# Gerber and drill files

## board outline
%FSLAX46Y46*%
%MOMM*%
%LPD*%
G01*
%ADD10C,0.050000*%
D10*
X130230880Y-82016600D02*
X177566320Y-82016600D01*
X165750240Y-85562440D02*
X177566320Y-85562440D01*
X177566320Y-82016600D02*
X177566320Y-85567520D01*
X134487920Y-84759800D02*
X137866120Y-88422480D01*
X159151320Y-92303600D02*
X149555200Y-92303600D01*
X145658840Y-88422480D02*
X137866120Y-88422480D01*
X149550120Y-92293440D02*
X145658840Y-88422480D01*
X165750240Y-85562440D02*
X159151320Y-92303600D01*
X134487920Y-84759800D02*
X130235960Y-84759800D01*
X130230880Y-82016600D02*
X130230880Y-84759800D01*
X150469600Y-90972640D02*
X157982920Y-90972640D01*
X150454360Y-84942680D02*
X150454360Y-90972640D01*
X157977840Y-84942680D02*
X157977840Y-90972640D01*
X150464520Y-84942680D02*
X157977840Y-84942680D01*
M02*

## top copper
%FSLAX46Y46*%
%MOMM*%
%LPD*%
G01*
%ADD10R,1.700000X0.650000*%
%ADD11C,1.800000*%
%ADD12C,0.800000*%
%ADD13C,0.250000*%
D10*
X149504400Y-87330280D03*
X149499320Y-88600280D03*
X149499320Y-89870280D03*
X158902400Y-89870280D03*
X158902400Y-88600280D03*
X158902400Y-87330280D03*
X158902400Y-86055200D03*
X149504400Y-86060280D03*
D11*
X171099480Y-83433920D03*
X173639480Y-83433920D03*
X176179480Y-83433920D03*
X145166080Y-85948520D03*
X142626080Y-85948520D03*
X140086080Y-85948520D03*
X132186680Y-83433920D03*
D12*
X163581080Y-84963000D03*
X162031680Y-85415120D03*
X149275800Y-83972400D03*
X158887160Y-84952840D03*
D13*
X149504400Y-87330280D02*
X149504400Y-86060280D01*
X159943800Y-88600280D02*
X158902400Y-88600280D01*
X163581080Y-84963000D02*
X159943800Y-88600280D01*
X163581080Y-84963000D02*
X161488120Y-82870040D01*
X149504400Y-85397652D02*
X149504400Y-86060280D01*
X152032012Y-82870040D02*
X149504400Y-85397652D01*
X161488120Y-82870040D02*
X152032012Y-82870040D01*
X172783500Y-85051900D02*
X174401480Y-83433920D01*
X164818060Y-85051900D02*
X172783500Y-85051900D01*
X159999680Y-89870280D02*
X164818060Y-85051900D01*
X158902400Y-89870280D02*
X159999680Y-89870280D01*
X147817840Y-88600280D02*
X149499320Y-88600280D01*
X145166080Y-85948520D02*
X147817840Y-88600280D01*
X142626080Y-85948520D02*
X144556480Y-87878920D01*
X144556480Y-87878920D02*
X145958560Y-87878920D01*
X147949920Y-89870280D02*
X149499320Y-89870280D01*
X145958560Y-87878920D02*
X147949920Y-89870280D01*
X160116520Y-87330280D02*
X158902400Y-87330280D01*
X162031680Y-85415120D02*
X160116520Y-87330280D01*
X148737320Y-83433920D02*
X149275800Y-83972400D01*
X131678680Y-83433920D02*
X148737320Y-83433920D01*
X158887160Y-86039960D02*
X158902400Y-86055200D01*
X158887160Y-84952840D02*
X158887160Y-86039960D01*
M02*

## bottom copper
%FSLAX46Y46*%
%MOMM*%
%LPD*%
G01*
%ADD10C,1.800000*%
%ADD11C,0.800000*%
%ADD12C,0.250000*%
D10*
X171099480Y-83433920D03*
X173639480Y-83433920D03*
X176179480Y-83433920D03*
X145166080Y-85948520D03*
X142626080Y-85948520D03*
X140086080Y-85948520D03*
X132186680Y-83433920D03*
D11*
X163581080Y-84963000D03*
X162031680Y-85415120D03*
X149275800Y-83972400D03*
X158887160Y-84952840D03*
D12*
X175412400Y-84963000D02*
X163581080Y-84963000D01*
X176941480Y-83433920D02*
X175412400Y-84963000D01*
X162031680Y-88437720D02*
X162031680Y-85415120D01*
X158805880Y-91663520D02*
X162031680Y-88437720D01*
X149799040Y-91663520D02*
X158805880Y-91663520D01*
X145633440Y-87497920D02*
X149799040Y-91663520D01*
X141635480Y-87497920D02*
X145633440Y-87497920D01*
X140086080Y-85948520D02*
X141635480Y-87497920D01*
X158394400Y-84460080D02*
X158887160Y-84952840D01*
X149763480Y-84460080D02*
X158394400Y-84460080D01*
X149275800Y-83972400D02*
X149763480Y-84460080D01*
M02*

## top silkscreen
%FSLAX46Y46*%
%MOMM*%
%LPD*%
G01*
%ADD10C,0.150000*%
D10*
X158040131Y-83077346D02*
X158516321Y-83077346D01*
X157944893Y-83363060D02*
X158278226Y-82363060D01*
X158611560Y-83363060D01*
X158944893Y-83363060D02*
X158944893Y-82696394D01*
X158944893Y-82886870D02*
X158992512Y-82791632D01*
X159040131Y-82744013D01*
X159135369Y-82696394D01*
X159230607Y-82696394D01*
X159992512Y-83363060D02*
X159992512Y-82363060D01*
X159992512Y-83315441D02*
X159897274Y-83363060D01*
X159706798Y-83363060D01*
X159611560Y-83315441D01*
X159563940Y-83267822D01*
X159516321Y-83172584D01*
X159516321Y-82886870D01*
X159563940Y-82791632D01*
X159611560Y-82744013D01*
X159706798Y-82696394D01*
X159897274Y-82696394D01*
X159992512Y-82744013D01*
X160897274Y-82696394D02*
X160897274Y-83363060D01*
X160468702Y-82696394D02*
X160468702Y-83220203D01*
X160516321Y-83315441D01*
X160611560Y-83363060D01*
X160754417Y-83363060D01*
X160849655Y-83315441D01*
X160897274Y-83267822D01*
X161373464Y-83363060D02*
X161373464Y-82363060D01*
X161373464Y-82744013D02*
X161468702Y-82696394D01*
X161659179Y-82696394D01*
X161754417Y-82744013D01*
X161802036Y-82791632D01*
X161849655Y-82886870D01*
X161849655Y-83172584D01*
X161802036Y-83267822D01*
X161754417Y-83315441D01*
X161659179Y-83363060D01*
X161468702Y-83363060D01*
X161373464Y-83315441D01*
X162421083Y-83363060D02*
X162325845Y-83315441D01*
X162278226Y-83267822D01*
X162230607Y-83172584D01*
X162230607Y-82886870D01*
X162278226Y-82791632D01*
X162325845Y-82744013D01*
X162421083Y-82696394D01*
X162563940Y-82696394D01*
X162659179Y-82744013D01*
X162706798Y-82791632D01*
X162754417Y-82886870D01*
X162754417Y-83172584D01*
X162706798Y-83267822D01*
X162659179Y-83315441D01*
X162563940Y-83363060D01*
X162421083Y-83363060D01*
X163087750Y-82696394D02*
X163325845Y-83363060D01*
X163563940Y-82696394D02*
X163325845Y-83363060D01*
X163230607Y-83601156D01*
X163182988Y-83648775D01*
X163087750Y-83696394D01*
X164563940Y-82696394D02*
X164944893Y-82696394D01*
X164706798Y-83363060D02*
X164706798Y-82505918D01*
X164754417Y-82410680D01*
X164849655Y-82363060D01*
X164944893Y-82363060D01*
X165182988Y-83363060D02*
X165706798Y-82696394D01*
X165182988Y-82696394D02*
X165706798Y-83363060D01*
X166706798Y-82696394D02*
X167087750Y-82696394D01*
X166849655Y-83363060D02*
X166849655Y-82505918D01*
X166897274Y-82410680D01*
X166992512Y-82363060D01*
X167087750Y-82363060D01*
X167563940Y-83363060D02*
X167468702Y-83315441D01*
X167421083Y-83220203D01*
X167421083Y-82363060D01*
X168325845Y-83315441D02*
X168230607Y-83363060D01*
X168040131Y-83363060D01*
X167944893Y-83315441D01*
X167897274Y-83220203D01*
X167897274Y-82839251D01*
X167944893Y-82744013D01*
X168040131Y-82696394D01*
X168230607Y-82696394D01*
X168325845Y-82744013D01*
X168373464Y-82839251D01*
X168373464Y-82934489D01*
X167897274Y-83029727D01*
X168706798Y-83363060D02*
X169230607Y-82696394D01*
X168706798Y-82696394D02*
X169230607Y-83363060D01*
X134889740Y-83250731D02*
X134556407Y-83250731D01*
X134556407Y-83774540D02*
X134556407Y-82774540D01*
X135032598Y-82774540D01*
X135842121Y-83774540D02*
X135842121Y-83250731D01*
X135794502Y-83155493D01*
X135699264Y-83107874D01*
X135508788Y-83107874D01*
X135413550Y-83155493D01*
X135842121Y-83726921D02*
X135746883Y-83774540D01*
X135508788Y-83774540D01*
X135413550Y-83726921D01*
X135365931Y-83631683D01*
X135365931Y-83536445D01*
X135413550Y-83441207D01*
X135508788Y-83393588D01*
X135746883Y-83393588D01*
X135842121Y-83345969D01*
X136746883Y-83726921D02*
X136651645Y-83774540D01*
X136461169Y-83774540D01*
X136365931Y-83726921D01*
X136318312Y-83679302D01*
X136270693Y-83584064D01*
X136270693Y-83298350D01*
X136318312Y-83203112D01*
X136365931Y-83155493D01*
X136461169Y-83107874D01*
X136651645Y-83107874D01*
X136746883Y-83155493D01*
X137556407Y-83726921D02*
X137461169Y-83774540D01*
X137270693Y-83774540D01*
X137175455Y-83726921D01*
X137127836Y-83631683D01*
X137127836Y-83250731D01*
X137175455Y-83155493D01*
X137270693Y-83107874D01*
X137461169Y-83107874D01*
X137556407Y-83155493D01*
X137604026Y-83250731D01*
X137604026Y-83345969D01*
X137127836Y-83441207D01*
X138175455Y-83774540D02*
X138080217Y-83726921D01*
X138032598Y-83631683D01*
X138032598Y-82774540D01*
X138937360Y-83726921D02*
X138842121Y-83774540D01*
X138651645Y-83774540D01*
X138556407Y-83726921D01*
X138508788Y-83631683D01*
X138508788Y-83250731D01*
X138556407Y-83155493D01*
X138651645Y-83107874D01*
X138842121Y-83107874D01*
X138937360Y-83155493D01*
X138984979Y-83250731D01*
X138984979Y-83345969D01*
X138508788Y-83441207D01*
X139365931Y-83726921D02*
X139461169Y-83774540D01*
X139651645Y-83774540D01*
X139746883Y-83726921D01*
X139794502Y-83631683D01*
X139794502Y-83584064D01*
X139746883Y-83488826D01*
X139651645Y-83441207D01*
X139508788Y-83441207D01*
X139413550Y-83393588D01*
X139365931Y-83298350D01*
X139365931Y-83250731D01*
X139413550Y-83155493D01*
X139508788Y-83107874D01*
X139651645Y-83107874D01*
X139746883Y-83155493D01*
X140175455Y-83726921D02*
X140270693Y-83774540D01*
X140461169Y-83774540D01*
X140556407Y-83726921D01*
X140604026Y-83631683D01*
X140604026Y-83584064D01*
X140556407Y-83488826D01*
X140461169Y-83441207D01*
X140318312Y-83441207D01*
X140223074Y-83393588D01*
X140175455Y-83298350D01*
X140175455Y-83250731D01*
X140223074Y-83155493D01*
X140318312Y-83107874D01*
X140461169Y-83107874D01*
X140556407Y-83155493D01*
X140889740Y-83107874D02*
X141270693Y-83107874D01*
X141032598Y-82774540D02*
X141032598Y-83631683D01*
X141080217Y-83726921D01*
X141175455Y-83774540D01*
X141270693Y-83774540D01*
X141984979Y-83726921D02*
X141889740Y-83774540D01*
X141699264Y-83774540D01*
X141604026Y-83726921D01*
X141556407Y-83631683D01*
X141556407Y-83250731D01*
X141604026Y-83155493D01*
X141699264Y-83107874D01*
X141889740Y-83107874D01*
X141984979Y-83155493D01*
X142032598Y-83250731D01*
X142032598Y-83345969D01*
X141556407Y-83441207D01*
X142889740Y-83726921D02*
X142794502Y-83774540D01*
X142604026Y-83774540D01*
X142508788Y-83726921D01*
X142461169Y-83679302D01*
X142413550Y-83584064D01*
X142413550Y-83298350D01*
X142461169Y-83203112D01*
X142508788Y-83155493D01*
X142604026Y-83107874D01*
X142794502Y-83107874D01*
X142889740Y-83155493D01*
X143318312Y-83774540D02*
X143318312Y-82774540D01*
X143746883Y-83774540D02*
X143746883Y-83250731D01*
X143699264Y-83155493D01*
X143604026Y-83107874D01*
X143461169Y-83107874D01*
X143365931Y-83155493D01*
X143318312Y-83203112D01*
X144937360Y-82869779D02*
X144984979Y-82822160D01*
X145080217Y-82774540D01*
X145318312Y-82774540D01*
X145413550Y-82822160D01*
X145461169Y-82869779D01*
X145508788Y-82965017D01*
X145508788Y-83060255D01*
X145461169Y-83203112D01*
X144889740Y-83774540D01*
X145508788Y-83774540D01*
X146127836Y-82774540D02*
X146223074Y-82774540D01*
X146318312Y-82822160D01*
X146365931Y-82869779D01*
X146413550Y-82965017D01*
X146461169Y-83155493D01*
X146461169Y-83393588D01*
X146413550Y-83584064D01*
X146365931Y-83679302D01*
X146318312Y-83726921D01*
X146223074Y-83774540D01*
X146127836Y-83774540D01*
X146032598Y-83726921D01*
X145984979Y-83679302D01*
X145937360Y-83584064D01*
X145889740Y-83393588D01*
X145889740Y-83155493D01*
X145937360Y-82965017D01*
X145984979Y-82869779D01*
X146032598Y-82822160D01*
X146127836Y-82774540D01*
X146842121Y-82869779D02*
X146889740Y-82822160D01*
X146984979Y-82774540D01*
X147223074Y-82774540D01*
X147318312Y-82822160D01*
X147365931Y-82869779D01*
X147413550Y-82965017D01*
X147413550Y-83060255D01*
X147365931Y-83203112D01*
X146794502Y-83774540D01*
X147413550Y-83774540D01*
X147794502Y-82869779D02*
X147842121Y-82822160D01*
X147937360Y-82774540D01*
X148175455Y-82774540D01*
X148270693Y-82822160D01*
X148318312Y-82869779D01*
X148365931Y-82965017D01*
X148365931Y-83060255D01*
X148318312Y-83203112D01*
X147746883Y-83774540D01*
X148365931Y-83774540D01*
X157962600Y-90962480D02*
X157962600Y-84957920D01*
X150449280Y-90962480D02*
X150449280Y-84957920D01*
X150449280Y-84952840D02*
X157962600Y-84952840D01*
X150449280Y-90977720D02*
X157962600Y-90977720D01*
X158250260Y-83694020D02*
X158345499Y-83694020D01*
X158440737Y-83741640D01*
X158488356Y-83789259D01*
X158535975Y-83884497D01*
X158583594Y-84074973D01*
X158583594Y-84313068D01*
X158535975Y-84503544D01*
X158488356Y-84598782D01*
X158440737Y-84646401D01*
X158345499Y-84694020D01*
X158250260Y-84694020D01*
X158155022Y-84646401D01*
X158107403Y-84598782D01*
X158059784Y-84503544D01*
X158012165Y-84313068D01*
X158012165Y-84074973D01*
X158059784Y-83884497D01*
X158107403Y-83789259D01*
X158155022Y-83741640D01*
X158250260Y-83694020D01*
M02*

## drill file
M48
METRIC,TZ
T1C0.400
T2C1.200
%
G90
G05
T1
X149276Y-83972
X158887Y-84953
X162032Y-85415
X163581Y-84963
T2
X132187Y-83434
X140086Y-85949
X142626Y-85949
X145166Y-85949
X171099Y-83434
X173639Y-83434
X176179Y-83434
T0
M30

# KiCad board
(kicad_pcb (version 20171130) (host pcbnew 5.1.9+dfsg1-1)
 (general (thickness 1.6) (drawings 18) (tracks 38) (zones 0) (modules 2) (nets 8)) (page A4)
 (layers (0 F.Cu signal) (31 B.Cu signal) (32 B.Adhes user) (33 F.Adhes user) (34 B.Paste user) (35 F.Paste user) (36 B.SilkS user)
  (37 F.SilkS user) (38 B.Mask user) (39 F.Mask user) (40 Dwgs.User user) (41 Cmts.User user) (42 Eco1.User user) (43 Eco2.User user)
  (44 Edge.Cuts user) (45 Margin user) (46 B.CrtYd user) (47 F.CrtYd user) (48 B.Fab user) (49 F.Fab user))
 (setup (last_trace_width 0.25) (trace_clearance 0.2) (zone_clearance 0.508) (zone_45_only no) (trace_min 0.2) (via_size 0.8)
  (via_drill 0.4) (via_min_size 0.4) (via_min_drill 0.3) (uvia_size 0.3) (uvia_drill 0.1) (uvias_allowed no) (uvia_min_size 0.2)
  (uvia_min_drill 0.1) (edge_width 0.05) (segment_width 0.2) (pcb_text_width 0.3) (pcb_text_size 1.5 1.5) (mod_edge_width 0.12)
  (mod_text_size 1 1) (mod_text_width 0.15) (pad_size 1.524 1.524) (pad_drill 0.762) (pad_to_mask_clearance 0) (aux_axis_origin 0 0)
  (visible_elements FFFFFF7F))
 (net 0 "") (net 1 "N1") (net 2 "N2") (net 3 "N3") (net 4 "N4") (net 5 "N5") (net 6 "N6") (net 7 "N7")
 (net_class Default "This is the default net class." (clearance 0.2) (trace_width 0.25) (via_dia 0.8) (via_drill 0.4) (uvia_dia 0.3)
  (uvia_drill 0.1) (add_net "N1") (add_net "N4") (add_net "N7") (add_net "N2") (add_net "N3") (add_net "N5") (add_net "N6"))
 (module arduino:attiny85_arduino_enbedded (layer F.Cu) (at 154.2034 87.96528)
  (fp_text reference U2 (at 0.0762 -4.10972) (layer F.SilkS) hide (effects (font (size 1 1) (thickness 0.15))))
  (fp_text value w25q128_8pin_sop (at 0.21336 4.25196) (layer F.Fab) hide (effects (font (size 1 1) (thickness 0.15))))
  (fp_line (start 3.7592 2.9972) (end 3.7592 -3.00736) (layer F.SilkS) (width 0.15))
  (fp_line (start -3.75412 2.9972) (end -3.75412 -3.00736) (layer F.SilkS) (width 0.15))
  (fp_line (start -3.75412 -3.01244) (end 3.7592 -3.01244) (layer F.SilkS) (width 0.15))
  (fp_line (start -3.75412 3.01244) (end 3.7592 3.01244) (layer F.SilkS) (width 0.15))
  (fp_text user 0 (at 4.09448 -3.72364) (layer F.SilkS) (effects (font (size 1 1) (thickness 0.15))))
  (pad 7 smd rect (at -4.699 -0.635) (size 1.7 0.65) (layers F.Cu F.Paste F.Mask) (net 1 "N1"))
  (pad 6 smd rect (at -4.70408 0.635) (size 1.7 0.65) (layers F.Cu F.Paste F.Mask) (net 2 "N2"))
  (pad 5 smd rect (at -4.70408 1.905) (size 1.7 0.65) (layers F.Cu F.Paste F.Mask) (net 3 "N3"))
  (pad 4 smd rect (at 4.699 1.905) (size 1.7 0.65) (layers F.Cu F.Paste F.Mask) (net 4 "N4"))
  (pad 3 smd rect (at 4.699 0.635) (size 1.7 0.65) (layers F.Cu F.Paste F.Mask) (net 1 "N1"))
  (pad 2 smd rect (at 4.699 -0.635) (size 1.7 0.65) (layers F.Cu F.Paste F.Mask) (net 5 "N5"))
  (pad 1 smd rect (at 4.699 -1.91008) (size 1.7 0.65) (layers F.Cu F.Paste F.Mask) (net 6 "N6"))
  (pad 8 smd rect (at -4.699 -1.905) (size 1.7 0.65) (layers F.Cu F.Paste F.Mask) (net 1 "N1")))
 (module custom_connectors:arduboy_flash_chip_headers (layer F.Cu) (at 154.15768 91.94292)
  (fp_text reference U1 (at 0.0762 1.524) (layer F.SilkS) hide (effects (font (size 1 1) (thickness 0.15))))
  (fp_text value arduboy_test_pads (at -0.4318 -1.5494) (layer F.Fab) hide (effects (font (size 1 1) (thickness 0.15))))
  (pad 3 thru_hole circle (at 16.9418 -8.509) (size 1.8 1.8) (drill 1.2) (layers *.Cu *.Mask) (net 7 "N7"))
  (pad 2 thru_hole circle (at 19.4818 -8.509) (size 1.8 1.8) (drill 1.2) (layers *.Cu *.Mask) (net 4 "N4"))
  (pad 1 thru_hole circle (at 22.0218 -8.509) (size 1.8 1.8) (drill 1.2) (layers *.Cu *.Mask) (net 1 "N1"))
  (pad 4 thru_hole circle (at -8.9916 -5.9944) (size 1.8 1.8) (drill 1.2) (layers *.Cu *.Mask) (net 2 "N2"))
  (pad 5 thru_hole circle (at -11.5316 -5.9944) (size 1.8 1.8) (drill 1.2) (layers *.Cu *.Mask) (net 3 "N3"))
  (pad 6 thru_hole circle (at -14.0716 -5.9944) (size 1.8 1.8) (drill 1.2) (layers *.Cu *.Mask) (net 5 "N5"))
  (pad 7 thru_hole circle (at -21.971 -8.509) (size 1.8 1.8) (drill 1.2) (layers *.Cu *.Mask) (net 6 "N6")))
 (gr_line (start 130.23088 82.0166) (end 177.56632 82.0166) (layer Edge.Cuts) (width 0.05))
 (gr_line (start 165.75024 85.56244) (end 177.56632 85.56244) (layer Edge.Cuts) (width 0.05))
 (gr_line (start 177.56632 82.0166) (end 177.56632 85.56752) (layer Edge.Cuts) (width 0.05))
 (gr_line (start 134.48792 84.7598) (end 137.86612 88.42248) (layer Edge.Cuts) (width 0.05))
 (gr_line (start 159.15132 92.3036) (end 149.5552 92.3036) (layer Edge.Cuts) (width 0.05))
 (gr_line (start 145.65884 88.42248) (end 137.86612 88.42248) (layer Edge.Cuts) (width 0.05))
 (gr_line (start 149.55012 92.29344) (end 145.65884 88.42248) (layer Edge.Cuts) (width 0.05))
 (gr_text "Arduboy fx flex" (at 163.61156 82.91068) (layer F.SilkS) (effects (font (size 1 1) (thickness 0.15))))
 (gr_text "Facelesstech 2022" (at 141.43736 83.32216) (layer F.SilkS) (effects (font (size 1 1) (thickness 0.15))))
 (gr_line (start 165.75024 85.56244) (end 159.15132 92.3036) (layer Edge.Cuts) (width 0.05))
 (gr_line (start 134.48792 84.7598) (end 130.23596 84.7598) (layer Edge.Cuts) (width 0.05))
 (gr_line (start 130.23088 82.0166) (end 130.23088 84.7598) (layer Edge.Cuts) (width 0.05))
 (gr_line (start 150.4696 90.97264) (end 157.98292 90.97264) (layer Edge.Cuts) (width 0.05))
 (gr_line (start 150.45436 84.94268) (end 150.45436 90.97264) (layer Edge.Cuts) (width 0.05))
 (gr_line (start 157.97784 84.94268) (end 157.97784 90.97264) (layer Edge.Cuts) (width 0.05))
 (gr_line (start 150.46452 84.94268) (end 157.97784 84.94268) (layer Edge.Cuts) (width 0.05))
 (segment (start 149.5044 87.33028) (end 149.5044 86.06028) (width 0.25) (layer F.Cu) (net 1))
 (via (at 163.58108 84.963) (size 0.8) (drill 0.4) (layers F.Cu B.Cu) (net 1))
 (segment (start 175.4124 84.963) (end 163.58108 84.963) (width 0.25) (layer B.Cu) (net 1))
 (segment (start 176.94148 83.43392) (end 175.4124 84.963) (width 0.25) (layer B.Cu) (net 1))
 (segment (start 159.9438 88.60028) (end 158.9024 88.60028) (width 0.25) (layer F.Cu) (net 1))
 (segment (start 163.58108 84.963) (end 159.9438 88.60028) (width 0.25) (layer F.Cu) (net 1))
 (segment (start 163.58108 84.963) (end 161.48812 82.87004) (width 0.25) (layer F.Cu) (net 1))
 (segment (start 149.5044 85.397652) (end 149.5044 86.06028) (width 0.25) (layer F.Cu) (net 1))
 (segment (start 152.032012 82.87004) (end 149.5044 85.397652) (width 0.25) (layer F.Cu) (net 1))
 (segment (start 161.48812 82.87004) (end 152.032012 82.87004) (width 0.25) (layer F.Cu) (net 1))
 (segment (start 172.7835 85.0519) (end 174.40148 83.43392) (width 0.25) (layer F.Cu) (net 4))
 (segment (start 164.81806 85.0519) (end 172.7835 85.0519) (width 0.25) (layer F.Cu) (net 4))
 (segment (start 159.99968 89.87028) (end 164.81806 85.0519) (width 0.25) (layer F.Cu) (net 4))
 (segment (start 158.9024 89.87028) (end 159.99968 89.87028) (width 0.25) (layer F.Cu) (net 4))
 (segment (start 147.81784 88.60028) (end 149.49932 88.60028) (width 0.25) (layer F.Cu) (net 2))
 (segment (start 145.16608 85.94852) (end 147.81784 88.60028) (width 0.25) (layer F.Cu) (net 2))
 (segment (start 142.62608 85.94852) (end 144.55648 87.87892) (width 0.25) (layer F.Cu) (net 3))
 (segment (start 144.55648 87.87892) (end 145.95856 87.87892) (width 0.25) (layer F.Cu) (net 3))
 (segment (start 147.94992 89.87028) (end 149.49932 89.87028) (width 0.25) (layer F.Cu) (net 3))
 (segment (start 145.95856 87.87892) (end 147.94992 89.87028) (width 0.25) (layer F.Cu) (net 3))
 (via (at 162.03168 85.41512) (size 0.8) (drill 0.4) (layers F.Cu B.Cu) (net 5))
 (segment (start 160.11652 87.33028) (end 158.9024 87.33028) (width 0.25) (layer F.Cu) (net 5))
 (segment (start 162.03168 85.41512) (end 160.11652 87.33028) (width 0.25) (layer F.Cu) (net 5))
 (segment (start 162.03168 88.43772) (end 162.03168 85.41512) (width 0.25) (layer B.Cu) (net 5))
 (segment (start 158.80588 91.66352) (end 162.03168 88.43772) (width 0.25) (layer B.Cu) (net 5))
 (segment (start 149.79904 91.66352) (end 158.80588 91.66352) (width 0.25) (layer B.Cu) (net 5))
 (segment (start 145.63344 87.49792) (end 149.79904 91.66352) (width 0.25) (layer B.Cu) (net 5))
 (segment (start 141.63548 87.49792) (end 145.63344 87.49792) (width 0.25) (layer B.Cu) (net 5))
 (segment (start 140.08608 85.94852) (end 141.63548 87.49792) (width 0.25) (layer B.Cu) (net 5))
 (via (at 149.2758 83.9724) (size 0.8) (drill 0.4) (layers F.Cu B.Cu) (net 6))
 (segment (start 148.73732 83.43392) (end 149.2758 83.9724) (width 0.25) (layer F.Cu) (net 6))
 (segment (start 131.67868 83.43392) (end 148.73732 83.43392) (width 0.25) (layer F.Cu) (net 6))
 (via (at 158.88716 84.95284) (size 0.8) (drill 0.4) (layers F.Cu B.Cu) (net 6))
 (segment (start 158.88716 86.03996) (end 158.9024 86.0552) (width 0.25) (layer F.Cu) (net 6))
 (segment (start 158.88716 84.95284) (end 158.88716 86.03996) (width 0.25) (layer F.Cu) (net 6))
 (segment (start 158.3944 84.46008) (end 158.88716 84.95284) (width 0.25) (layer B.Cu) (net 6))
 (segment (start 149.76348 84.46008) (end 158.3944 84.46008) (width 0.25) (layer B.Cu) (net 6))
 (segment (start 149.2758 83.9724) (end 149.76348 84.46008) (width 0.25) (layer B.Cu) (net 6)))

